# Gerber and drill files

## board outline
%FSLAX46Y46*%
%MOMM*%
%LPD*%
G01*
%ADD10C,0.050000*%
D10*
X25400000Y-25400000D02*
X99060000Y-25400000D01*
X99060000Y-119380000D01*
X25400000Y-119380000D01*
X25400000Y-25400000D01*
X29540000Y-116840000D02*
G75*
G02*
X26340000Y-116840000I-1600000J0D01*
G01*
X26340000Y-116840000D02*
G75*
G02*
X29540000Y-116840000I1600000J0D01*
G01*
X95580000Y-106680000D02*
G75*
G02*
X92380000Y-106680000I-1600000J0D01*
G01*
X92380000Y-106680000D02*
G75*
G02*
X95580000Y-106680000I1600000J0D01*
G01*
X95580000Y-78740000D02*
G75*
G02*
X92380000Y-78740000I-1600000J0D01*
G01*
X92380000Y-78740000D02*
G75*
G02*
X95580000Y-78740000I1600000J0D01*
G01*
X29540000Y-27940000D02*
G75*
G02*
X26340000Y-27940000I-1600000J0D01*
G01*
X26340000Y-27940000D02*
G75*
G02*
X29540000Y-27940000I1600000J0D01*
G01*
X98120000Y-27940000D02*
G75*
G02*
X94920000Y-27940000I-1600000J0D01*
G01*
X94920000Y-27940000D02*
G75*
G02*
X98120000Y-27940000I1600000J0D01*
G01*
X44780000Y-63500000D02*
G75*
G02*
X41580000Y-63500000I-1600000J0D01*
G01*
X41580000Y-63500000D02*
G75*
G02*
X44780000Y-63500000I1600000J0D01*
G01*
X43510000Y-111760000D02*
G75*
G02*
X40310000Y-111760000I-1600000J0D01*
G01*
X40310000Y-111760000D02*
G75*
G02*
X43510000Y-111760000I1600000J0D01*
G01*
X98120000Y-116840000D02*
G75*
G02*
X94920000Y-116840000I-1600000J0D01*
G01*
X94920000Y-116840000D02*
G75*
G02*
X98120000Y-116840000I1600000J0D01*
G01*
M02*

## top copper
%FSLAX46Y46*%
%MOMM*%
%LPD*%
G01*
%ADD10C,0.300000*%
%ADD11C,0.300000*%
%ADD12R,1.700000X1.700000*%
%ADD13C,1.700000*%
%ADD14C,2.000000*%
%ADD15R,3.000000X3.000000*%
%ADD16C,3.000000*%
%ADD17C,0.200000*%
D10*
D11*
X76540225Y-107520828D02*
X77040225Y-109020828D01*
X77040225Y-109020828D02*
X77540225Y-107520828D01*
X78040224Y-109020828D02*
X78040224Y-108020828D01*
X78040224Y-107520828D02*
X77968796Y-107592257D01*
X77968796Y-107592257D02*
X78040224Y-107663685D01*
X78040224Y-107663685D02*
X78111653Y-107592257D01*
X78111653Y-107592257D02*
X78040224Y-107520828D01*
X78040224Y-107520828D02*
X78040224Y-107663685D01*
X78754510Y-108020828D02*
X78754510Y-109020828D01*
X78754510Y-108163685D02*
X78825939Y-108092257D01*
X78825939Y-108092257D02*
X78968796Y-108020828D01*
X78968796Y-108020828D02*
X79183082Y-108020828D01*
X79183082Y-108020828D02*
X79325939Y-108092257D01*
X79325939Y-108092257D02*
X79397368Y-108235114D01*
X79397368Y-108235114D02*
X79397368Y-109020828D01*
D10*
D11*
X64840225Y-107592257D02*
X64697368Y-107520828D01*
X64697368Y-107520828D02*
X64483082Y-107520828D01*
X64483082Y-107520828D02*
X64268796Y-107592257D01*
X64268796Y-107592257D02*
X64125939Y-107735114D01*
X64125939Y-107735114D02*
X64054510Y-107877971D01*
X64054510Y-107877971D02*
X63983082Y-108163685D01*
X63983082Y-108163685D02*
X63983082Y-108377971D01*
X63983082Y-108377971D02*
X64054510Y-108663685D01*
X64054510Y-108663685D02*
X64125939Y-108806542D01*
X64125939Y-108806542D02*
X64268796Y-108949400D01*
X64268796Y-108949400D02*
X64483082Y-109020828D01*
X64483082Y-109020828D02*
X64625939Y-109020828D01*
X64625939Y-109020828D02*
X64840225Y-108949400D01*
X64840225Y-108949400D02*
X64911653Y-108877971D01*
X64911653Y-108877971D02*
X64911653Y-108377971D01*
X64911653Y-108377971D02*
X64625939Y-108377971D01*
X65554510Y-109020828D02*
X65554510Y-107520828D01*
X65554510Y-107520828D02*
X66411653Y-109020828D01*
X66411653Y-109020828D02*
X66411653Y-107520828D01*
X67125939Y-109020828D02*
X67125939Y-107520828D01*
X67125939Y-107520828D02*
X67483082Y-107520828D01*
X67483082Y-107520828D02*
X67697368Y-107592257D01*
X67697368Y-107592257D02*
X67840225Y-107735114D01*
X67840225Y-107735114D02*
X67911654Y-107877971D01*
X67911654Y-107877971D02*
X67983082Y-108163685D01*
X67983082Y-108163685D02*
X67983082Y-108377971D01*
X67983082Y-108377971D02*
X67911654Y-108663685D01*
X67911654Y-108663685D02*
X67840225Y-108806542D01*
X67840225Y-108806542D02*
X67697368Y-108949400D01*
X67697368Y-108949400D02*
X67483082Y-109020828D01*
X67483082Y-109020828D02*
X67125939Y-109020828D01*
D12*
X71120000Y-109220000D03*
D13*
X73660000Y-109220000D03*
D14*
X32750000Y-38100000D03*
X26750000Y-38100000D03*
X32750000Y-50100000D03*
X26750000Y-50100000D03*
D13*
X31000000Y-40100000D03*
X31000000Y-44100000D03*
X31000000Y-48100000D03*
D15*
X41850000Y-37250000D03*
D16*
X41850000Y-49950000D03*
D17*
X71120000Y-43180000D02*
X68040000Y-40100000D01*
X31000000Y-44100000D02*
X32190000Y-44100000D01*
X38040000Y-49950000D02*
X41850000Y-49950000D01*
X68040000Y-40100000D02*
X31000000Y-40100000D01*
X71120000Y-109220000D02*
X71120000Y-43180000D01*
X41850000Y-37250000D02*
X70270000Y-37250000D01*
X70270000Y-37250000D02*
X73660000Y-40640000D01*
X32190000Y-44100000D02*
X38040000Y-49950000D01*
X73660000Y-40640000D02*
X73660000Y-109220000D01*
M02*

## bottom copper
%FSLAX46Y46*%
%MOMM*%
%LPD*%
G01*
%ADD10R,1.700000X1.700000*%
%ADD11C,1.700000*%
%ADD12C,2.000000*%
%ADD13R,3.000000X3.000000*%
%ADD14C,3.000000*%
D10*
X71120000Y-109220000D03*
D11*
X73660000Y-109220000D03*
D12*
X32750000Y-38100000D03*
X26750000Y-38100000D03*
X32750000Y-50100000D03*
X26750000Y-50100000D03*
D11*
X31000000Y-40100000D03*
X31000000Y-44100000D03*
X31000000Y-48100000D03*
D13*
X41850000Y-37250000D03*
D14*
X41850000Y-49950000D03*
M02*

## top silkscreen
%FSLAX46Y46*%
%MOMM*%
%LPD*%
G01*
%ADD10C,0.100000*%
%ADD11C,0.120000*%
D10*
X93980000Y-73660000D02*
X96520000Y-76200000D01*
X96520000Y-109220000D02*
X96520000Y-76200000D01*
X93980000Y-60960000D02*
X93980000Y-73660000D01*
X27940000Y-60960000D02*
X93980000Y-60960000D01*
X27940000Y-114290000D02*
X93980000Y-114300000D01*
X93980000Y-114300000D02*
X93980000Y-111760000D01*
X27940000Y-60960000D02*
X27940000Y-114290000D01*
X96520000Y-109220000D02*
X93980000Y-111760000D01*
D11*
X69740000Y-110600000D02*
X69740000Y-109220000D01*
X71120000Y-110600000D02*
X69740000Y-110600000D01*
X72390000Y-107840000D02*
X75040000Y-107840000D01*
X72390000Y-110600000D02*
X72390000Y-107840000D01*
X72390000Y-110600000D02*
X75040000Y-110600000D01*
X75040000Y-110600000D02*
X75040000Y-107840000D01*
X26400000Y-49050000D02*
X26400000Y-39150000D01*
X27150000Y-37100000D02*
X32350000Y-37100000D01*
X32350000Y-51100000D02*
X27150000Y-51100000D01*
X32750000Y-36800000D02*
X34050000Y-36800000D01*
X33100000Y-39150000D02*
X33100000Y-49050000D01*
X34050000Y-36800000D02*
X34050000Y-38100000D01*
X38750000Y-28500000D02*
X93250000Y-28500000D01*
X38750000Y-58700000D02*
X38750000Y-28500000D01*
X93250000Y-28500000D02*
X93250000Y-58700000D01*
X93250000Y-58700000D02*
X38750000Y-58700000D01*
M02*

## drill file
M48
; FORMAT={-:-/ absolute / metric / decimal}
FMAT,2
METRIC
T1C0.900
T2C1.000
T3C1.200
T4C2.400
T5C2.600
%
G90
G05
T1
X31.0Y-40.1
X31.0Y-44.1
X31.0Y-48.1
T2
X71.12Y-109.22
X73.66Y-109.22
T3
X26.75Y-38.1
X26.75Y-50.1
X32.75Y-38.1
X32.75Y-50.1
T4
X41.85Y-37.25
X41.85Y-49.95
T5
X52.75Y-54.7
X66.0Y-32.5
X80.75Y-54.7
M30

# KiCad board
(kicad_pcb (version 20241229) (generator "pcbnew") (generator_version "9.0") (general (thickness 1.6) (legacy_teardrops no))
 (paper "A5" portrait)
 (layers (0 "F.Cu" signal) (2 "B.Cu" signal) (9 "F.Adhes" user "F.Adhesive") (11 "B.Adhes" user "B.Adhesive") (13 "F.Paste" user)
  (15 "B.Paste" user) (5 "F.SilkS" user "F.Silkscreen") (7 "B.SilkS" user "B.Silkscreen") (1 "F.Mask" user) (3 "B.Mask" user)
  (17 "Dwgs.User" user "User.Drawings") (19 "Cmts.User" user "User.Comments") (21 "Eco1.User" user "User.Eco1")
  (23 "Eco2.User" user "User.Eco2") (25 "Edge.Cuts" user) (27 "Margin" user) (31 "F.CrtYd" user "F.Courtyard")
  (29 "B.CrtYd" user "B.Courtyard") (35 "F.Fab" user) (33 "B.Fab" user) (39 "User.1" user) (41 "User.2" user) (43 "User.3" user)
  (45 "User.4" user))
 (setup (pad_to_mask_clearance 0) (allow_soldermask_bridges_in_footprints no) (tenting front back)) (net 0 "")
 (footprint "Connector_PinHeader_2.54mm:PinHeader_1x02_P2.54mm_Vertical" (layer "F.Cu") (at 71.12 109.22 90)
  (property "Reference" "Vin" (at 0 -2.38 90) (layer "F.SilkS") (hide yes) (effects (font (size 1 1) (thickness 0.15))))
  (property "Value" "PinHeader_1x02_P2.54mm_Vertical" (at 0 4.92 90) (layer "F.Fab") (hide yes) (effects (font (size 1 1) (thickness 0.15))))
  (fp_line (start -1.38 -1.38) (end 0 -1.38) (stroke (width 0.12) (type solid)) (layer "F.SilkS"))
  (fp_line (start -1.38 0) (end -1.38 -1.38) (stroke (width 0.12) (type solid)) (layer "F.SilkS"))
  (fp_line (start 1.38 1.27) (end 1.38 3.92) (stroke (width 0.12) (type solid)) (layer "F.SilkS"))
  (fp_line (start -1.38 1.27) (end 1.38 1.27) (stroke (width 0.12) (type solid)) (layer "F.SilkS"))
  (fp_line (start -1.38 1.27) (end -1.38 3.92) (stroke (width 0.12) (type solid)) (layer "F.SilkS"))
  (fp_line (start -1.38 3.92) (end 1.38 3.92) (stroke (width 0.12) (type solid)) (layer "F.SilkS"))
  (pad "1" thru_hole rect (at 0 0 90) (size 1.7 1.7) (drill 1) (layers "*.Cu" "*.Mask") (remove_unused_layers no))
  (pad "2" thru_hole circle (at 0 2.54 90) (size 1.7 1.7) (drill 1) (layers "*.Cu" "*.Mask") (remove_unused_layers no)))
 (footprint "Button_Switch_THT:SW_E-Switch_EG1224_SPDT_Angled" (layer "F.Cu") (at 31 40.1 -90)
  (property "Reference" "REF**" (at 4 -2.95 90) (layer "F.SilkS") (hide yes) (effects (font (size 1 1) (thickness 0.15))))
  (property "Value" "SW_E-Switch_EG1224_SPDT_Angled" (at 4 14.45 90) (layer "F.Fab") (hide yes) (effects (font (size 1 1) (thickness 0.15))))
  (fp_line (start 8.95 4.6) (end -0.95 4.6) (stroke (width 0.12) (type solid)) (layer "F.SilkS"))
  (fp_line (start -3 3.85) (end -3 -1.35) (stroke (width 0.12) (type solid)) (layer "F.SilkS"))
  (fp_line (start 11 -1.35) (end 11 3.85) (stroke (width 0.12) (type solid)) (layer "F.SilkS"))
  (fp_line (start -3.3 -1.75) (end -3.3 -3.05) (stroke (width 0.12) (type solid)) (layer "F.SilkS"))
  (fp_line (start -0.95 -2.1) (end 8.95 -2.1) (stroke (width 0.12) (type solid)) (layer "F.SilkS"))
  (fp_line (start -3.3 -3.05) (end -2 -3.05) (stroke (width 0.12) (type solid)) (layer "F.SilkS"))
  (pad "" thru_hole circle (at -2 -1.75 270) (size 2 2) (drill 1.2) (layers "*.Cu" "*.Mask") (remove_unused_layers no))
  (pad "" thru_hole circle (at -2 4.25 270) (size 2 2) (drill 1.2) (layers "*.Cu" "*.Mask") (remove_unused_layers no))
  (pad "" thru_hole circle (at 10 -1.75 270) (size 2 2) (drill 1.2) (layers "*.Cu" "*.Mask") (remove_unused_layers no))
  (pad "" thru_hole circle (at 10 4.25 270) (size 2 2) (drill 1.2) (layers "*.Cu" "*.Mask") (remove_unused_layers no))
  (pad "1" thru_hole circle (at 0 0 270) (size 1.7 1.7) (drill 0.9) (layers "*.Cu" "*.Mask") (remove_unused_layers no))
  (pad "2" thru_hole circle (at 4 0 270) (size 1.7 1.7) (drill 0.9) (layers "*.Cu" "*.Mask") (remove_unused_layers no))
  (pad "3" thru_hole circle (at 8 0 270) (size 1.7 1.7) (drill 0.9) (layers "*.Cu" "*.Mask") (remove_unused_layers no)))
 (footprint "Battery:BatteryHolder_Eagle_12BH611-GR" (layer "F.Cu") (at 41.85 37.25 180)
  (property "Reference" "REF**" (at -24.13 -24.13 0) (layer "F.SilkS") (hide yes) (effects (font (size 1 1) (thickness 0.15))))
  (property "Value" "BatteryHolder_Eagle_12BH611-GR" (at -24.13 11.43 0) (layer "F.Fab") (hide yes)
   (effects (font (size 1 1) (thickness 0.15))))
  (fp_line (start 3.1 8.75) (end -51.4 8.75) (stroke (width 0.12) (type solid)) (layer "F.SilkS"))
  (fp_line (start 3.1 -21.45) (end 3.1 8.75) (stroke (width 0.12) (type solid)) (layer "F.SilkS"))
  (fp_line (start -51.4 8.75) (end -51.4 -21.45) (stroke (width 0.12) (type solid)) (layer "F.SilkS"))
  (fp_line (start -51.4 -21.45) (end 3.1 -21.45) (stroke (width 0.12) (type solid)) (layer "F.SilkS"))
  (pad "" np_thru_hole circle (at -38.9 -17.45 180) (size 2.6 2.6) (drill 2.6) (layers "*.Cu" "*.Mask"))
  (pad "" np_thru_hole circle (at -24.15 4.75 180) (size 2.6 2.6) (drill 2.6) (layers "*.Cu" "*.Mask"))
  (pad "" np_thru_hole circle (at -10.9 -17.45 180) (size 2.6 2.6) (drill 2.6) (layers "*.Cu" "*.Mask"))
  (pad "1" thru_hole rect (at 0 0 180) (size 3 3) (drill 2.4) (layers "*.Cu" "*.Mask") (remove_unused_layers no))
  (pad "2" thru_hole circle (at 0 -12.7 180) (size 3 3) (drill 2.4) (layers "*.Cu" "*.Mask") (remove_unused_layers no)))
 (gr_line (start 93.98 73.66) (end 96.52 76.2) (stroke (width 0.1) (type solid)) (layer "F.SilkS"))
 (gr_line (start 96.52 109.22) (end 96.52 76.2) (stroke (width 0.1) (type solid)) (layer "F.SilkS"))
 (gr_line (start 93.98 60.96) (end 93.98 73.66) (stroke (width 0.1) (type solid)) (layer "F.SilkS"))
 (gr_line (start 27.94 60.96) (end 93.98 60.96) (stroke (width 0.1) (type solid)) (layer "F.SilkS"))
 (gr_line (start 27.94 114.29) (end 93.98 114.3) (stroke (width 0.1) (type solid)) (layer "F.SilkS"))
 (gr_line (start 93.98 114.3) (end 93.98 111.76) (stroke (width 0.1) (type solid)) (layer "F.SilkS"))
 (gr_line (start 27.94 60.96) (end 27.94 114.29) (stroke (width 0.1) (type solid)) (layer "F.SilkS"))
 (gr_line (start 96.52 109.22) (end 93.98 111.76) (stroke (width 0.1) (type default)) (layer "F.SilkS"))
 (gr_rect (start 25.4 25.4) (end 99.06 119.38) (stroke (width 0.05) (type default)) (fill no) (layer "Edge.Cuts"))
 (gr_circle (center 27.94 116.84) (end 29.54 116.84) (stroke (width 0.05) (type solid)) (fill no) (layer "Edge.Cuts"))
 (gr_circle (center 93.98 106.68) (end 95.58 106.68) (stroke (width 0.05) (type solid)) (fill no) (layer "Edge.Cuts"))
 (gr_circle (center 93.98 78.74) (end 95.58 78.74) (stroke (width 0.05) (type solid)) (fill no) (layer "Edge.Cuts"))
 (gr_circle (center 27.94 27.94) (end 29.54 27.94) (stroke (width 0.05) (type solid)) (fill no) (layer "Edge.Cuts"))
 (gr_circle (center 96.52 27.94) (end 98.12 27.94) (stroke (width 0.05) (type solid)) (fill no) (layer "Edge.Cuts"))
 (gr_circle (center 43.18 63.5) (end 44.78 63.5) (stroke (width 0.05) (type solid)) (fill no) (layer "Edge.Cuts"))
 (gr_circle (center 41.91 111.76) (end 43.51 111.76) (stroke (width 0.05) (type solid)) (fill no) (layer "Edge.Cuts"))
 (gr_circle (center 96.52 116.84) (end 98.12 116.84) (stroke (width 0.05) (type solid)) (fill no) (layer "Edge.Cuts"))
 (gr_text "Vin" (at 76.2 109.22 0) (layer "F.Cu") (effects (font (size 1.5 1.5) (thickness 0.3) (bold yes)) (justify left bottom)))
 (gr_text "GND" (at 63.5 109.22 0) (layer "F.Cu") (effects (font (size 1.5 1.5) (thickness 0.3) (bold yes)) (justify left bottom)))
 (segment (start 71.12 43.18) (end 68.04 40.1) (width 0.2) (layer "F.Cu") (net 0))
 (segment (start 31 44.1) (end 32.19 44.1) (width 0.2) (layer "F.Cu") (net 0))
 (segment (start 38.04 49.95) (end 41.85 49.95) (width 0.2) (layer "F.Cu") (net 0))
 (segment (start 68.04 40.1) (end 31 40.1) (width 0.2) (layer "F.Cu") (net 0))
 (segment (start 71.12 109.22) (end 71.12 43.18) (width 0.2) (layer "F.Cu") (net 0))
 (segment (start 41.85 37.25) (end 70.27 37.25) (width 0.2) (layer "F.Cu") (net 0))
 (segment (start 70.27 37.25) (end 73.66 40.64) (width 0.2) (layer "F.Cu") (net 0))
 (segment (start 32.19 44.1) (end 38.04 49.95) (width 0.2) (layer "F.Cu") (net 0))
 (segment (start 73.66 40.64) (end 73.66 109.22) (width 0.2) (layer "F.Cu") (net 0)))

